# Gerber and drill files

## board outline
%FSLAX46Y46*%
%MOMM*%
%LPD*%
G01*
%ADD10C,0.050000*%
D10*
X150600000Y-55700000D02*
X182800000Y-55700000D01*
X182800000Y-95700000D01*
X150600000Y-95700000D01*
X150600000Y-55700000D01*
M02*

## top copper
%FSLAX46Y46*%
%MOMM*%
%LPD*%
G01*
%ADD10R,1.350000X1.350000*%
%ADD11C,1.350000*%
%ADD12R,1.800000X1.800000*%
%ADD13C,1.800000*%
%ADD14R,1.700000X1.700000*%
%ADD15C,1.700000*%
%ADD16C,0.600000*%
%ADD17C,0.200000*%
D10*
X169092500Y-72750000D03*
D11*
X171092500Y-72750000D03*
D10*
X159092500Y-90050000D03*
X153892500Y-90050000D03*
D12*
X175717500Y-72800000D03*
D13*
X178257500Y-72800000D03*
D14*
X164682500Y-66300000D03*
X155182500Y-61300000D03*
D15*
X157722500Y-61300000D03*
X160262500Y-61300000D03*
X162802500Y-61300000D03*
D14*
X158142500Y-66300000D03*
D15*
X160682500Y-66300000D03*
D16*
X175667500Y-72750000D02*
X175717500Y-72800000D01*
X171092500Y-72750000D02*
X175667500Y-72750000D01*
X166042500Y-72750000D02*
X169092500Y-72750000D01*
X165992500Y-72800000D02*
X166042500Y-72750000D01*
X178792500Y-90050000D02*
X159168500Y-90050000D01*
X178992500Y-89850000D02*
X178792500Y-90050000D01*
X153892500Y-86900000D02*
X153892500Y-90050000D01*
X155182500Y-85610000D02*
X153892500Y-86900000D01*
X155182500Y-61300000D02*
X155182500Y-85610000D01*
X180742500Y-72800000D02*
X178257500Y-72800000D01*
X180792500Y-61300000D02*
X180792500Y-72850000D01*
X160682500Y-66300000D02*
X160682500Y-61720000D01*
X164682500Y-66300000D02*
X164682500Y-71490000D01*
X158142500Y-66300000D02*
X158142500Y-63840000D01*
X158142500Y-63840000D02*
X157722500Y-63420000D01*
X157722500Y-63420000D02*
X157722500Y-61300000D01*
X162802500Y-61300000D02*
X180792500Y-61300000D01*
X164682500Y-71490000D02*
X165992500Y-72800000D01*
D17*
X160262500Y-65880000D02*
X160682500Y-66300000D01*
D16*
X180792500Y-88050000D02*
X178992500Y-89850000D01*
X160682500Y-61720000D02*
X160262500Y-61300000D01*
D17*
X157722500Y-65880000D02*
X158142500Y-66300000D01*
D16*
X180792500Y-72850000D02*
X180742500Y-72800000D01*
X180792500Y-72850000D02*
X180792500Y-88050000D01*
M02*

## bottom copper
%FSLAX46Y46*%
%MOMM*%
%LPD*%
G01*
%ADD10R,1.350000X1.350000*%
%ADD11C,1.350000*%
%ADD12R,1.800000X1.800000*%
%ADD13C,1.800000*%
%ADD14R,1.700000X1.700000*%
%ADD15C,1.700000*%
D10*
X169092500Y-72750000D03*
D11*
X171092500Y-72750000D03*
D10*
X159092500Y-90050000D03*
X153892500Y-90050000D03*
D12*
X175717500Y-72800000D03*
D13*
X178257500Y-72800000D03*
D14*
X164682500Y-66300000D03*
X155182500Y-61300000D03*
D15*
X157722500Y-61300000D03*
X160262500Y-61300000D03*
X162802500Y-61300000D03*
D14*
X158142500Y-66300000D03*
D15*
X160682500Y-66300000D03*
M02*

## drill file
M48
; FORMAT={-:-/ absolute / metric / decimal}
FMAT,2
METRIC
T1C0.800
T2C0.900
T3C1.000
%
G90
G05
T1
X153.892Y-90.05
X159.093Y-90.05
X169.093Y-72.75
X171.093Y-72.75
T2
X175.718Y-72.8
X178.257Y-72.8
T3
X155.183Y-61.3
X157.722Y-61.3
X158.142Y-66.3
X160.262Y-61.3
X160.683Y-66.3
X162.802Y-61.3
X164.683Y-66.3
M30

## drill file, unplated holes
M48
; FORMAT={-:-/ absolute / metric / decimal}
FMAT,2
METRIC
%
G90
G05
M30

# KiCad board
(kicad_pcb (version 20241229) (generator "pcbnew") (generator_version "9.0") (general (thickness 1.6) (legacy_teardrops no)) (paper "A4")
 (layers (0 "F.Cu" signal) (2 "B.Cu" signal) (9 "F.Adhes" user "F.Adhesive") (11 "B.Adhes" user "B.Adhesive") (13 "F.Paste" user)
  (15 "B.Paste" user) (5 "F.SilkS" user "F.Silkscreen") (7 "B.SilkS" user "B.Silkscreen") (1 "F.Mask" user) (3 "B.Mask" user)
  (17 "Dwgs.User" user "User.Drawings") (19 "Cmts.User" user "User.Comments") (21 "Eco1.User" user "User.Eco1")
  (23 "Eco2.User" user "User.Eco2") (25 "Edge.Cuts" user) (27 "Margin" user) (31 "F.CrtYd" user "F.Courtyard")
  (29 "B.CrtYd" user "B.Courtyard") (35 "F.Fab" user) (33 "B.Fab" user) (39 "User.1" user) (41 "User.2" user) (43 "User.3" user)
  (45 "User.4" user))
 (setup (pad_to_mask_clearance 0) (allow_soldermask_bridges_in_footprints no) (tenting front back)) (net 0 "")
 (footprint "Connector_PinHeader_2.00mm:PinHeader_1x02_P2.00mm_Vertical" (layer "F.Cu") (at 169.0925 72.75 90)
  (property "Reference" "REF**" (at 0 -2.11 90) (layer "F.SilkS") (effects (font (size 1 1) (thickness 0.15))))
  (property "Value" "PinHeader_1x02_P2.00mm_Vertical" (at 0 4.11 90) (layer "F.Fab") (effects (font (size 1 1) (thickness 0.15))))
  (pad "1" thru_hole rect (at 0 0 90) (size 1.35 1.35) (drill 0.8) (layers "*.Cu" "*.Mask") (remove_unused_layers no))
  (pad "2" thru_hole circle (at 0 2 90) (size 1.35 1.35) (drill 0.8) (layers "*.Cu" "*.Mask") (remove_unused_layers no)))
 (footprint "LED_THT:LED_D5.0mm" (layer "F.Cu") (at 175.7175 72.8)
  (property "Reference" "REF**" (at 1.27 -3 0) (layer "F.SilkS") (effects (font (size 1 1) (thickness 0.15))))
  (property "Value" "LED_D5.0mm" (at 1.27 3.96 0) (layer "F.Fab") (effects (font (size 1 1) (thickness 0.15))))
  (pad "1" thru_hole rect (at 0 0) (size 1.8 1.8) (drill 0.9) (layers "*.Cu" "*.Mask") (remove_unused_layers no))
  (pad "2" thru_hole circle (at 2.54 0) (size 1.8 1.8) (drill 0.9) (layers "*.Cu" "*.Mask") (remove_unused_layers no)))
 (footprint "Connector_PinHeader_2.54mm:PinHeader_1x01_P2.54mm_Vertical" (layer "F.Cu") (at 164.6825 66.3)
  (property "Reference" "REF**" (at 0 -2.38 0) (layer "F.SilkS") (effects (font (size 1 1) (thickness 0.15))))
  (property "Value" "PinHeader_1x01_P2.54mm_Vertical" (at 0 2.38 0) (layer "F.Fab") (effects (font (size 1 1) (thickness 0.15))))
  (pad "1" thru_hole rect (at 0 0) (size 1.7 1.7) (drill 1) (layers "*.Cu" "*.Mask") (remove_unused_layers no)))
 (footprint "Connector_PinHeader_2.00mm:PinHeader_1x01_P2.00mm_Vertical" (layer "F.Cu") (at 153.8925 90.05)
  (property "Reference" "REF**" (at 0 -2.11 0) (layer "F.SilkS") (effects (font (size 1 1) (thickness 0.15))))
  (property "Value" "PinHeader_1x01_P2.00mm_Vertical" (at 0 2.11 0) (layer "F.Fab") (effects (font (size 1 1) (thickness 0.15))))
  (pad "1" thru_hole rect (at 0 0) (size 1.35 1.35) (drill 0.8) (layers "*.Cu" "*.Mask") (remove_unused_layers no)))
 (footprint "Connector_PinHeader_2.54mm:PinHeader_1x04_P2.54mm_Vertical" (layer "F.Cu") (at 155.1825 61.3 90)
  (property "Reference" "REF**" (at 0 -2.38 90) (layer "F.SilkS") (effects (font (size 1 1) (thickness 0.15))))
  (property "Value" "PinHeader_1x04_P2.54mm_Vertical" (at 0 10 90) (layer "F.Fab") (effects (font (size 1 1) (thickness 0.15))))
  (pad "1" thru_hole rect (at 0 0 90) (size 1.7 1.7) (drill 1) (layers "*.Cu" "*.Mask") (remove_unused_layers no))
  (pad "2" thru_hole circle (at 0 2.54 90) (size 1.7 1.7) (drill 1) (layers "*.Cu" "*.Mask") (remove_unused_layers no))
  (pad "3" thru_hole circle (at 0 5.08 90) (size 1.7 1.7) (drill 1) (layers "*.Cu" "*.Mask") (remove_unused_layers no))
  (pad "4" thru_hole circle (at 0 7.62 90) (size 1.7 1.7) (drill 1) (layers "*.Cu" "*.Mask") (remove_unused_layers no)))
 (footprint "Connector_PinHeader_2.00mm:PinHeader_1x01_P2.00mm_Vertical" (layer "F.Cu") (at 159.0925 90.05)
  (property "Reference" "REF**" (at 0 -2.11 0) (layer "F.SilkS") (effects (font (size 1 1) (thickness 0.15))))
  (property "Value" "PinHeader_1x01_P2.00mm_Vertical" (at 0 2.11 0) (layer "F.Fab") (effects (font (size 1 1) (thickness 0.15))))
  (pad "1" thru_hole rect (at 0 0) (size 1.35 1.35) (drill 0.8) (layers "*.Cu" "*.Mask") (remove_unused_layers no)))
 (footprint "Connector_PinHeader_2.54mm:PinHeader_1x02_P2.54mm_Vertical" (layer "F.Cu") (at 158.1425 66.3 90)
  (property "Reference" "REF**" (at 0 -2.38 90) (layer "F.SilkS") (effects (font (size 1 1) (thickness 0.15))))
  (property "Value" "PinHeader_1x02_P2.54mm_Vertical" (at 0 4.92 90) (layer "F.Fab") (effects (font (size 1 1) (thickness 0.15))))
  (pad "1" thru_hole rect (at 0 0 90) (size 1.7 1.7) (drill 1) (layers "*.Cu" "*.Mask") (remove_unused_layers no))
  (pad "2" thru_hole circle (at 0 2.54 90) (size 1.7 1.7) (drill 1) (layers "*.Cu" "*.Mask") (remove_unused_layers no)))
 (gr_rect (start 150.6 55.7) (end 182.8 95.7) (stroke (width 0.05) (type default)) (fill no) (layer "Edge.Cuts"))
 (segment (start 180.7425 72.8) (end 178.2575 72.8) (width 0.6) (layer "F.Cu") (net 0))
 (segment (start 165.9925 72.8) (end 166.0425 72.75) (width 0.6) (layer "F.Cu") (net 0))
 (segment (start 175.6675 72.75) (end 175.7175 72.8) (width 0.6) (layer "F.Cu") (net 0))
 (segment (start 180.7925 61.3) (end 180.7925 72.85) (width 0.6) (layer "F.Cu") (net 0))
 (segment (start 160.6825 66.3) (end 160.6825 61.72) (width 0.6) (layer "F.Cu") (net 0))
 (segment (start 171.0925 72.75) (end 175.6675 72.75) (width 0.6) (layer "F.Cu") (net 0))
 (segment (start 164.6825 66.3) (end 164.6825 71.49) (width 0.6) (layer "F.Cu") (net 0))
 (segment (start 158.1425 66.3) (end 158.1425 63.84) (width 0.6) (layer "F.Cu") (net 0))
 (segment (start 158.1425 63.84) (end 157.7225 63.42) (width 0.6) (layer "F.Cu") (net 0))
 (segment (start 157.7225 63.42) (end 157.7225 61.3) (width 0.6) (layer "F.Cu") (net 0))
 (segment (start 155.1825 85.61) (end 153.8925 86.9) (width 0.6) (layer "F.Cu") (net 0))
 (segment (start 178.7925 90.05) (end 159.1685 90.05) (width 0.6) (layer "F.Cu") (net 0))
 (segment (start 153.8925 86.9) (end 153.8925 90.05) (width 0.6) (layer "F.Cu") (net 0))
 (segment (start 166.0425 72.75) (end 169.0925 72.75) (width 0.6) (layer "F.Cu") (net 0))
 (segment (start 162.8025 61.3) (end 180.7925 61.3) (width 0.6) (layer "F.Cu") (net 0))
 (segment (start 164.6825 71.49) (end 165.9925 72.8) (width 0.6) (layer "F.Cu") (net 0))
 (segment (start 160.2625 65.88) (end 160.6825 66.3) (width 0.2) (layer "F.Cu") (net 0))
 (segment (start 180.7925 88.05) (end 178.9925 89.85) (width 0.6) (layer "F.Cu") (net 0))
 (segment (start 178.9925 89.85) (end 178.7925 90.05) (width 0.6) (layer "F.Cu") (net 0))
 (segment (start 160.6825 61.72) (end 160.2625 61.3) (width 0.6) (layer "F.Cu") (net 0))
 (segment (start 157.7225 65.88) (end 158.1425 66.3) (width 0.2) (layer "F.Cu") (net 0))
 (segment (start 155.1825 61.3) (end 155.1825 85.61) (width 0.6) (layer "F.Cu") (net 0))
 (segment (start 180.7925 72.85) (end 180.7425 72.8) (width 0.6) (layer "F.Cu") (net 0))
 (segment (start 180.7925 72.85) (end 180.7925 88.05) (width 0.6) (layer "F.Cu") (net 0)))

